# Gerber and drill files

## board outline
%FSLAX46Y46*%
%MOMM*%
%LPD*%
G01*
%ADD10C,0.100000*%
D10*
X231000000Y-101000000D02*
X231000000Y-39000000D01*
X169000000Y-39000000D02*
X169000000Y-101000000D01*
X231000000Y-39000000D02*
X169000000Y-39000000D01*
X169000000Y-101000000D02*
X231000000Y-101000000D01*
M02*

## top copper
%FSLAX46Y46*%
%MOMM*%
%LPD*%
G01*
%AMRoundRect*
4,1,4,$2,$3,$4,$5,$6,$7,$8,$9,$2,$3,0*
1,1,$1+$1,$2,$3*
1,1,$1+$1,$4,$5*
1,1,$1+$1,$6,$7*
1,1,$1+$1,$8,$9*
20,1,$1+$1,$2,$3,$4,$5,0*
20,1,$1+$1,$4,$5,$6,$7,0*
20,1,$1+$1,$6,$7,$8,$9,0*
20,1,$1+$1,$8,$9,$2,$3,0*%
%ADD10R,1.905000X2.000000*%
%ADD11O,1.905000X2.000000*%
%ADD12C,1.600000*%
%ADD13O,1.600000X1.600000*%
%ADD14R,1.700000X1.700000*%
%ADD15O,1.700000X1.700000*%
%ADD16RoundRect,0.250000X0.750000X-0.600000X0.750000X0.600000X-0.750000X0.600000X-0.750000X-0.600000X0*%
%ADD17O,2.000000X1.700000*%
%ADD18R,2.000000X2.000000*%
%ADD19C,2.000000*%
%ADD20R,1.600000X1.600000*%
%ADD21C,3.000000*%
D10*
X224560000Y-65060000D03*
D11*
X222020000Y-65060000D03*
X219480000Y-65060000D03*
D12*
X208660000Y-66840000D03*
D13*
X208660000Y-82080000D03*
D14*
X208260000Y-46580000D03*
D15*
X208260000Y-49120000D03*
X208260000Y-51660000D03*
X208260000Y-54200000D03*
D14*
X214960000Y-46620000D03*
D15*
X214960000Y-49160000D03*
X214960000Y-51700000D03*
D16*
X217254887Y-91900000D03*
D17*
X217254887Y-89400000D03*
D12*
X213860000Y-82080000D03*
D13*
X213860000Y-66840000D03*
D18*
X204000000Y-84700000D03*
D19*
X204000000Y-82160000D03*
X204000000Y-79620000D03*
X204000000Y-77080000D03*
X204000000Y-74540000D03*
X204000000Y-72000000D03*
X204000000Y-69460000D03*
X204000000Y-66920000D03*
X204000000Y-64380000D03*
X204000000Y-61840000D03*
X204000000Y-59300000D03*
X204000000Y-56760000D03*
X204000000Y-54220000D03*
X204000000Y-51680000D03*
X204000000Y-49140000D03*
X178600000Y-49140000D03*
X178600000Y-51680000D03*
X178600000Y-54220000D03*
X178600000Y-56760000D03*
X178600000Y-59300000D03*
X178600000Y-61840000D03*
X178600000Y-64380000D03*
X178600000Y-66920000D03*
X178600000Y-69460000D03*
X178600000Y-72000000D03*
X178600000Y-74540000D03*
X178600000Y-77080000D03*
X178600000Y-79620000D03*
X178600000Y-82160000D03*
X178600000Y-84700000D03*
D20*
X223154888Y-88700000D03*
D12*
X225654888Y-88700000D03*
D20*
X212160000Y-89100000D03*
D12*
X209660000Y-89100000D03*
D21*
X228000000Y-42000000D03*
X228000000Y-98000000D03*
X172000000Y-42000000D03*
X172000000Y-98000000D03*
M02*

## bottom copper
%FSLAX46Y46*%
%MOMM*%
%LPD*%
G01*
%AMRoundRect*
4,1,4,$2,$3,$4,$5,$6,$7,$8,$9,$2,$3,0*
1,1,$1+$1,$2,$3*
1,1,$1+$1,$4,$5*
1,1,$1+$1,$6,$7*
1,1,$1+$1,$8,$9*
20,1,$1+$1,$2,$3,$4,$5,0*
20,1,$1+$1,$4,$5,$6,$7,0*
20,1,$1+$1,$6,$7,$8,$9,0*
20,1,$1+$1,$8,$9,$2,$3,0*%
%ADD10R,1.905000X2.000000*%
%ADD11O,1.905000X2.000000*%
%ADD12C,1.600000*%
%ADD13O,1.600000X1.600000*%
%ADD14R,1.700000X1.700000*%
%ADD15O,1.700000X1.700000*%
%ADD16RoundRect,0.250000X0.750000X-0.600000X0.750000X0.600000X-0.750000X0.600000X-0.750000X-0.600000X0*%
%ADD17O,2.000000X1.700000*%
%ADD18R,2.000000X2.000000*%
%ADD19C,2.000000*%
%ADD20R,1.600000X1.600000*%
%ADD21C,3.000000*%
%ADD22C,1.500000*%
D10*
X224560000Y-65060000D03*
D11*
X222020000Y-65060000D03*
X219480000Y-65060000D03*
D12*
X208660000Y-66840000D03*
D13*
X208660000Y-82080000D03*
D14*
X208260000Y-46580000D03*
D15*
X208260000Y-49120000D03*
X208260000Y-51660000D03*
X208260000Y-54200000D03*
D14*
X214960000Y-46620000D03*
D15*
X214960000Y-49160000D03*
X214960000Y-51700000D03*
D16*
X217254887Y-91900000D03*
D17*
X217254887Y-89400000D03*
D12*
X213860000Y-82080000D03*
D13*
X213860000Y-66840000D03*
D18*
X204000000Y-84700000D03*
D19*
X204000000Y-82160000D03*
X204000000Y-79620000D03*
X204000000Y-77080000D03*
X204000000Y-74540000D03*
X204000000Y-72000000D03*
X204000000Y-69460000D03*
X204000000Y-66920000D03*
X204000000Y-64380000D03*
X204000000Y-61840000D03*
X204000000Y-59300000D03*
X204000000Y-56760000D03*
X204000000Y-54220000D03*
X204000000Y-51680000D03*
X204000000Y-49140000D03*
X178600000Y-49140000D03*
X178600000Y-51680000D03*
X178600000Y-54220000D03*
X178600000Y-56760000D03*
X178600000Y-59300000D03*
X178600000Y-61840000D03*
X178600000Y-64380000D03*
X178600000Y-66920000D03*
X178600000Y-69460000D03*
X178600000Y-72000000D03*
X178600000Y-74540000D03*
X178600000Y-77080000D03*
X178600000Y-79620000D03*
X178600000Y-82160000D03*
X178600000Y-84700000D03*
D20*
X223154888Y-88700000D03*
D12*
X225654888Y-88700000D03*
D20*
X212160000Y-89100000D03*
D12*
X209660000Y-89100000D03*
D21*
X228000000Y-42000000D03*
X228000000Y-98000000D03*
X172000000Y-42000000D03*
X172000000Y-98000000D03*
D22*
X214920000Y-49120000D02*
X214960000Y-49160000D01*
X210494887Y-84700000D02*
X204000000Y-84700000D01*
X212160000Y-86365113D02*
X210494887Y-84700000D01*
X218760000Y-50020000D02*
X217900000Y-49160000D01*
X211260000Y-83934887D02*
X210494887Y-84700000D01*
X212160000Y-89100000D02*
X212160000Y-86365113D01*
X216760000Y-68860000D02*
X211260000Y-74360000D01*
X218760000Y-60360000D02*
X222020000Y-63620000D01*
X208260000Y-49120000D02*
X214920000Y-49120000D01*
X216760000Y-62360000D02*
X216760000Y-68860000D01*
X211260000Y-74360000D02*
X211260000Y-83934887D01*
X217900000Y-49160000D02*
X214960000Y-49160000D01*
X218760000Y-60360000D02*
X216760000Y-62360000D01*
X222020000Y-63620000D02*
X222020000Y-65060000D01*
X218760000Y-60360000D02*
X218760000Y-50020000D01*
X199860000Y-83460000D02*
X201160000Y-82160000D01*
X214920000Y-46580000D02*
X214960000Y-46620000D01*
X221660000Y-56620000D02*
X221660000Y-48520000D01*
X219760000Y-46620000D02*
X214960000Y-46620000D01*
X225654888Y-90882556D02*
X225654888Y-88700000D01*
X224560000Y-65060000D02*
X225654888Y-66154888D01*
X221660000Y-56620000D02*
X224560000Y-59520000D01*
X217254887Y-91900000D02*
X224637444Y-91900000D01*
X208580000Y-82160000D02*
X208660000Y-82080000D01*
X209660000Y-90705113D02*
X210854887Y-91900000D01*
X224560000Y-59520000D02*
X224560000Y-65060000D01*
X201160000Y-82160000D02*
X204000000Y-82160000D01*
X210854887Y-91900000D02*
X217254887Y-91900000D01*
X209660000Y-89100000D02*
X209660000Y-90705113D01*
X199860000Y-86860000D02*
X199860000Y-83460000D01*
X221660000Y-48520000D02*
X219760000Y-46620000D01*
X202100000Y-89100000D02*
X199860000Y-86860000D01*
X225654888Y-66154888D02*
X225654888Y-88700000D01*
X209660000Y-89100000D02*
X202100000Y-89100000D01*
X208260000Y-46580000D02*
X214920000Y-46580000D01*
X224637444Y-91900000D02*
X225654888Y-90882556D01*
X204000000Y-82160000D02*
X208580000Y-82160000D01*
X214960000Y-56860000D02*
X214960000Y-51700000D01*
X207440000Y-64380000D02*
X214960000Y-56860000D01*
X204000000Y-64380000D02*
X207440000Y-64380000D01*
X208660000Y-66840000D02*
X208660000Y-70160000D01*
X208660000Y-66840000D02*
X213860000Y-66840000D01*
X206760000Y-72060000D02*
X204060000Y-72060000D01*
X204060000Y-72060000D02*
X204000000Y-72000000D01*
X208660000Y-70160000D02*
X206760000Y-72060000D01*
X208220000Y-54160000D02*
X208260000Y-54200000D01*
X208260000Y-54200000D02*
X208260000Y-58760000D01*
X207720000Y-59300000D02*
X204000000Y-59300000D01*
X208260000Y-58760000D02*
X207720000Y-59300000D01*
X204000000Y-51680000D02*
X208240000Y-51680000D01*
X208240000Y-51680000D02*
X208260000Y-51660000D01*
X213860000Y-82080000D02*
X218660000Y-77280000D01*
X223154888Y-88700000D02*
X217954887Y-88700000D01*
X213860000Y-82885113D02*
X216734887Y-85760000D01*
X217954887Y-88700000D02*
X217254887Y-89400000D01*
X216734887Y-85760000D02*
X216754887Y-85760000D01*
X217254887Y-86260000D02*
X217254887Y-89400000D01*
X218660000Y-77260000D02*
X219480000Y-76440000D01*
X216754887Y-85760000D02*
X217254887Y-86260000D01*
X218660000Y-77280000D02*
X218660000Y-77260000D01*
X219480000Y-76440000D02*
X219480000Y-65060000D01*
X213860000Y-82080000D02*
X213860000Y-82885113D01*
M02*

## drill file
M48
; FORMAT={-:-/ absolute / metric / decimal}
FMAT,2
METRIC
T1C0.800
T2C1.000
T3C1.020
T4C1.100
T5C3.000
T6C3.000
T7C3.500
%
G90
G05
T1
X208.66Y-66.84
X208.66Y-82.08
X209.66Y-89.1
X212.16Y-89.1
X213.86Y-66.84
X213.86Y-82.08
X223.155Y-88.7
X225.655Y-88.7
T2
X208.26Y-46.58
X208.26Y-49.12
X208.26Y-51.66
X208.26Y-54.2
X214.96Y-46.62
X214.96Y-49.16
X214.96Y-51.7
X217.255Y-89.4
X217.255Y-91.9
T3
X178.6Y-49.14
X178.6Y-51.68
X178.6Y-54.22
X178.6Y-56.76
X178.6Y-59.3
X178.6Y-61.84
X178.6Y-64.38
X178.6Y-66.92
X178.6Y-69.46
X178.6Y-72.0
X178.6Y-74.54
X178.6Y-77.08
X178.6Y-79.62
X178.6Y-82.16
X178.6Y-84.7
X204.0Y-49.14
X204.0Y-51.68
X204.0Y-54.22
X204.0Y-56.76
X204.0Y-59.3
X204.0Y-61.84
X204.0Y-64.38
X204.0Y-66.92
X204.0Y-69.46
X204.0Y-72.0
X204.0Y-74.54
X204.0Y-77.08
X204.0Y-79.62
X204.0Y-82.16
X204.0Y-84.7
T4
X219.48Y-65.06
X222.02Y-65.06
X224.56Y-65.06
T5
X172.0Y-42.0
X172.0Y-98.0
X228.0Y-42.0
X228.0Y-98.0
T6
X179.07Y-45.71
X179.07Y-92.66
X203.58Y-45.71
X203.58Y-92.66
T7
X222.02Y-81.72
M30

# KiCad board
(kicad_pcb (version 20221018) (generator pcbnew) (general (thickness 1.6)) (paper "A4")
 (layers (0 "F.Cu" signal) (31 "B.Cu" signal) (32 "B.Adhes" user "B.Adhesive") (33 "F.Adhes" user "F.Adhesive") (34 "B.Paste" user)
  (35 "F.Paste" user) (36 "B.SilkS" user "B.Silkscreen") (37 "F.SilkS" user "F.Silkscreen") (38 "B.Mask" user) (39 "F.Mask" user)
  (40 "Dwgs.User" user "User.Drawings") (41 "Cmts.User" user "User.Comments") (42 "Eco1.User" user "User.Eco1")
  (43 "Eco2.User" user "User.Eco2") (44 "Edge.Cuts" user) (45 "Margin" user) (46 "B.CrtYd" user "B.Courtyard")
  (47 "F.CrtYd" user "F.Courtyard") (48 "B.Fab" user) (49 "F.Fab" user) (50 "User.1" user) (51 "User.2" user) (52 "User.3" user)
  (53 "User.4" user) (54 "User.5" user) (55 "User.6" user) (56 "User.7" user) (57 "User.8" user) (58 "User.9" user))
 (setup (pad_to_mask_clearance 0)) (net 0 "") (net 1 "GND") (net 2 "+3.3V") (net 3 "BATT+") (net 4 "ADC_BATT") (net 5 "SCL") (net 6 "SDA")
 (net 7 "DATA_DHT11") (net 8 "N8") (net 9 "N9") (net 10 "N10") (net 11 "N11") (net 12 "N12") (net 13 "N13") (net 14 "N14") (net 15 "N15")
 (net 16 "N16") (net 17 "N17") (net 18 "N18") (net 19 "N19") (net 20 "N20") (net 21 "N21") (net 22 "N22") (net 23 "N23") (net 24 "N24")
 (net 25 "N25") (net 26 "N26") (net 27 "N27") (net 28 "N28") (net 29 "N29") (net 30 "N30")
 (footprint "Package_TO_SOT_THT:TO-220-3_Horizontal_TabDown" (layer "F.Cu") (at 224.56 65.06 180)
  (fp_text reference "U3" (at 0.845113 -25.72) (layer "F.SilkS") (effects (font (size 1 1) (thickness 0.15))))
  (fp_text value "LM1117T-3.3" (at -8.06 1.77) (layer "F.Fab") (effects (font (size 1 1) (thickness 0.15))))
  (pad "" np_thru_hole oval (at 2.54 -16.66 180) (size 3.5 3.5) (drill 3.5) (layers "*.Cu" "*.Mask"))
  (pad "1" thru_hole rect (at 0 0 180) (size 1.905 2) (drill 1.1) (layers "*.Cu" "*.Mask") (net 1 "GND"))
  (pad "2" thru_hole oval (at 2.54 0 180) (size 1.905 2) (drill 1.1) (layers "*.Cu" "*.Mask") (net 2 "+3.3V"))
  (pad "3" thru_hole oval (at 5.08 0 180) (size 1.905 2) (drill 1.1) (layers "*.Cu" "*.Mask") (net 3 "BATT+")))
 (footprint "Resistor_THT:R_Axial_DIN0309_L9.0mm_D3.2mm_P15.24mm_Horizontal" (layer "F.Cu") (at 208.66 66.84 -90)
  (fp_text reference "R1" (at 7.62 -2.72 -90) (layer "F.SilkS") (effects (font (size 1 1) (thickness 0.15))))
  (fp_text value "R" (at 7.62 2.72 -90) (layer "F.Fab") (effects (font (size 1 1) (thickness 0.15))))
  (pad "1" thru_hole circle (at 0 0 270) (size 1.6 1.6) (drill 0.8) (layers "*.Cu" "*.Mask") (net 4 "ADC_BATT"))
  (pad "2" thru_hole oval (at 15.24 0 270) (size 1.6 1.6) (drill 0.8) (layers "*.Cu" "*.Mask") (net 1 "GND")))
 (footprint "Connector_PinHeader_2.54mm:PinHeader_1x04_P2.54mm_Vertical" (layer "F.Cu") (at 208.26 46.58)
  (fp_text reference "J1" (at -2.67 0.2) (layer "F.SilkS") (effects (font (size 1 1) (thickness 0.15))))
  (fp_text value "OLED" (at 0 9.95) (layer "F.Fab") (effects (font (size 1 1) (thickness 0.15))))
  (pad "1" thru_hole rect (at 0 0) (size 1.7 1.7) (drill 1) (layers "*.Cu" "*.Mask") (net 1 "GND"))
  (pad "2" thru_hole oval (at 0 2.54) (size 1.7 1.7) (drill 1) (layers "*.Cu" "*.Mask") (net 2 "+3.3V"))
  (pad "3" thru_hole oval (at 0 5.08) (size 1.7 1.7) (drill 1) (layers "*.Cu" "*.Mask") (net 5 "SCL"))
  (pad "4" thru_hole oval (at 0 7.62) (size 1.7 1.7) (drill 1) (layers "*.Cu" "*.Mask") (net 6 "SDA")))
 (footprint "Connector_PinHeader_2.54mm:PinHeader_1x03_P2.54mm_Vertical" (layer "F.Cu") (at 214.96 46.62)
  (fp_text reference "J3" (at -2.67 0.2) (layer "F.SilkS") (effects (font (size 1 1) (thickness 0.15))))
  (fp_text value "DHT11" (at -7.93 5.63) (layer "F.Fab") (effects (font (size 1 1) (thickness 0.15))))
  (pad "1" thru_hole rect (at 0 0) (size 1.7 1.7) (drill 1) (layers "*.Cu" "*.Mask") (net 1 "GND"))
  (pad "2" thru_hole oval (at 0 2.54) (size 1.7 1.7) (drill 1) (layers "*.Cu" "*.Mask") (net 2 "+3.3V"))
  (pad "3" thru_hole oval (at 0 5.08) (size 1.7 1.7) (drill 1) (layers "*.Cu" "*.Mask") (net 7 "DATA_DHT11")))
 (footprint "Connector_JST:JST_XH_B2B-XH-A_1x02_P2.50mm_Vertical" (layer "F.Cu") (at 217.254887 91.9 90)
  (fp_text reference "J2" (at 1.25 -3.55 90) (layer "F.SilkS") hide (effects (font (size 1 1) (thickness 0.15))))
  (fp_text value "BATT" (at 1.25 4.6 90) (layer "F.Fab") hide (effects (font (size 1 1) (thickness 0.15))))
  (pad "1" thru_hole roundrect (at 0 0 90) (size 1.7 2) (drill 1) (layers "*.Cu" "*.Mask") (roundrect_rratio 0.1470588235) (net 1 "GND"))
  (pad "2" thru_hole oval (at 2.5 0 90) (size 1.7 2) (drill 1) (layers "*.Cu" "*.Mask") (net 3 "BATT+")))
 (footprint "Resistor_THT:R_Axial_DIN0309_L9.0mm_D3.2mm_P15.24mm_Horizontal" (layer "F.Cu") (at 213.86 82.08 90)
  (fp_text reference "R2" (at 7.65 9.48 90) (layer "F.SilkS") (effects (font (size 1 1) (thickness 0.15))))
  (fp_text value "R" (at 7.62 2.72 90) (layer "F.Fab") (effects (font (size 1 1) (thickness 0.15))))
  (pad "1" thru_hole circle (at 0 0 90) (size 1.6 1.6) (drill 0.8) (layers "*.Cu" "*.Mask") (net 3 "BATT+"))
  (pad "2" thru_hole oval (at 15.24 0 90) (size 1.6 1.6) (drill 0.8) (layers "*.Cu" "*.Mask") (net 4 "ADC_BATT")))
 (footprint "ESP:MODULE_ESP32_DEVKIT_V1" (layer "F.Cu") (at 191.3 69.185 180)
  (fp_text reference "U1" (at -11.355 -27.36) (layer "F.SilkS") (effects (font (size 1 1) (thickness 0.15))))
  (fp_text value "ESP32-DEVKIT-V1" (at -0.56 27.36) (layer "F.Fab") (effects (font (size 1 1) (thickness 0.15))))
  (pad "" np_thru_hole circle (at -12.28 -23.475 180) (size 3 3) (drill 3) (layers "*.Cu" "*.Mask"))
  (pad "" np_thru_hole circle (at -12.28 23.475 180) (size 3 3) (drill 3) (layers "*.Cu" "*.Mask"))
  (pad "" np_thru_hole circle (at 12.23 -23.475 180) (size 3 3) (drill 3) (layers "*.Cu" "*.Mask"))
  (pad "" np_thru_hole circle (at 12.23 23.475 180) (size 3 3) (drill 3) (layers "*.Cu" "*.Mask"))
  (pad "1" thru_hole rect (at -12.7 -15.515 180) (size 2 2) (drill 1.02) (layers "*.Cu" "*.Mask") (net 2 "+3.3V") (solder_mask_margin 0.102))
  (pad "2" thru_hole circle (at -12.7 -12.975 180) (size 2 2) (drill 1.02) (layers "*.Cu" "*.Mask") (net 1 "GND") (solder_mask_margin 0.102))
  (pad "3" thru_hole circle (at -12.7 -10.435 180) (size 2 2) (drill 1.02) (layers "*.Cu" "*.Mask") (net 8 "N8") (solder_mask_margin 0.102))
  (pad "4" thru_hole circle (at -12.7 -7.895 180) (size 2 2) (drill 1.02) (layers "*.Cu" "*.Mask") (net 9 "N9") (solder_mask_margin 0.102))
  (pad "5" thru_hole circle (at -12.7 -5.355 180) (size 2 2) (drill 1.02) (layers "*.Cu" "*.Mask") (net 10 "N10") (solder_mask_margin 0.102))
  (pad "6" thru_hole circle (at -12.7 -2.815 180) (size 2 2) (drill 1.02) (layers "*.Cu" "*.Mask") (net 4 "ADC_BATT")
   (solder_mask_margin 0.102))
  (pad "7" thru_hole circle (at -12.7 -0.275 180) (size 2 2) (drill 1.02) (layers "*.Cu" "*.Mask") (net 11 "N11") (solder_mask_margin 0.102))
  (pad "8" thru_hole circle (at -12.7 2.265 180) (size 2 2) (drill 1.02) (layers "*.Cu" "*.Mask") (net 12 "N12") (solder_mask_margin 0.102))
  (pad "9" thru_hole circle (at -12.7 4.805 180) (size 2 2) (drill 1.02) (layers "*.Cu" "*.Mask") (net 7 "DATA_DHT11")
   (solder_mask_margin 0.102))
  (pad "10" thru_hole circle (at -12.7 7.345 180) (size 2 2) (drill 1.02) (layers "*.Cu" "*.Mask") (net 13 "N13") (solder_mask_margin 0.102))
  (pad "11" thru_hole circle (at -12.7 9.885 180) (size 2 2) (drill 1.02) (layers "*.Cu" "*.Mask") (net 6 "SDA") (solder_mask_margin 0.102))
  (pad "12" thru_hole circle (at -12.7 12.425 180) (size 2 2) (drill 1.02) (layers "*.Cu" "*.Mask") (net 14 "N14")
   (solder_mask_margin 0.102))
  (pad "13" thru_hole circle (at -12.7 14.965 180) (size 2 2) (drill 1.02) (layers "*.Cu" "*.Mask") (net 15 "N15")
   (solder_mask_margin 0.102))
  (pad "14" thru_hole circle (at -12.7 17.505 180) (size 2 2) (drill 1.02) (layers "*.Cu" "*.Mask") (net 5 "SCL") (solder_mask_margin 0.102))
  (pad "15" thru_hole circle (at -12.7 20.045 180) (size 2 2) (drill 1.02) (layers "*.Cu" "*.Mask") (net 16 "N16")
   (solder_mask_margin 0.102))
  (pad "16" thru_hole circle (at 12.7 20.045 180) (size 2 2) (drill 1.02) (layers "*.Cu" "*.Mask") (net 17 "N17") (solder_mask_margin 0.102))
  (pad "17" thru_hole circle (at 12.7 17.505 180) (size 2 2) (drill 1.02) (layers "*.Cu" "*.Mask") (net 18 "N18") (solder_mask_margin 0.102))
  (pad "18" thru_hole circle (at 12.7 14.965 180) (size 2 2) (drill 1.02) (layers "*.Cu" "*.Mask") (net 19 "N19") (solder_mask_margin 0.102))
  (pad "19" thru_hole circle (at 12.7 12.425 180) (size 2 2) (drill 1.02) (layers "*.Cu" "*.Mask") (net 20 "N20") (solder_mask_margin 0.102))
  (pad "20" thru_hole circle (at 12.7 9.885 180) (size 2 2) (drill 1.02) (layers "*.Cu" "*.Mask") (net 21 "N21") (solder_mask_margin 0.102))
  (pad "21" thru_hole circle (at 12.7 7.345 180) (size 2 2) (drill 1.02) (layers "*.Cu" "*.Mask") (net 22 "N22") (solder_mask_margin 0.102))
  (pad "22" thru_hole circle (at 12.7 4.805 180) (size 2 2) (drill 1.02) (layers "*.Cu" "*.Mask") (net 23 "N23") (solder_mask_margin 0.102))
  (pad "23" thru_hole circle (at 12.7 2.265 180) (size 2 2) (drill 1.02) (layers "*.Cu" "*.Mask") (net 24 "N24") (solder_mask_margin 0.102))
  (pad "24" thru_hole circle (at 12.7 -0.275 180) (size 2 2) (drill 1.02) (layers "*.Cu" "*.Mask") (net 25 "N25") (solder_mask_margin 0.102))
  (pad "25" thru_hole circle (at 12.7 -2.815 180) (size 2 2) (drill 1.02) (layers "*.Cu" "*.Mask") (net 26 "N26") (solder_mask_margin 0.102))
  (pad "26" thru_hole circle (at 12.7 -5.355 180) (size 2 2) (drill 1.02) (layers "*.Cu" "*.Mask") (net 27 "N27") (solder_mask_margin 0.102))
  (pad "27" thru_hole circle (at 12.7 -7.895 180) (size 2 2) (drill 1.02) (layers "*.Cu" "*.Mask") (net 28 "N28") (solder_mask_margin 0.102))
  (pad "28" thru_hole circle (at 12.7 -10.435 180) (size 2 2) (drill 1.02) (layers "*.Cu" "*.Mask") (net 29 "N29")
   (solder_mask_margin 0.102))
  (pad "29" thru_hole circle (at 12.7 -12.975 180) (size 2 2) (drill 1.02) (layers "*.Cu" "*.Mask") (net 1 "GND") (solder_mask_margin 0.102))
  (pad "30" thru_hole circle (at 12.7 -15.515 180) (size 2 2) (drill 1.02) (layers "*.Cu" "*.Mask") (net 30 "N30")
   (solder_mask_margin 0.102))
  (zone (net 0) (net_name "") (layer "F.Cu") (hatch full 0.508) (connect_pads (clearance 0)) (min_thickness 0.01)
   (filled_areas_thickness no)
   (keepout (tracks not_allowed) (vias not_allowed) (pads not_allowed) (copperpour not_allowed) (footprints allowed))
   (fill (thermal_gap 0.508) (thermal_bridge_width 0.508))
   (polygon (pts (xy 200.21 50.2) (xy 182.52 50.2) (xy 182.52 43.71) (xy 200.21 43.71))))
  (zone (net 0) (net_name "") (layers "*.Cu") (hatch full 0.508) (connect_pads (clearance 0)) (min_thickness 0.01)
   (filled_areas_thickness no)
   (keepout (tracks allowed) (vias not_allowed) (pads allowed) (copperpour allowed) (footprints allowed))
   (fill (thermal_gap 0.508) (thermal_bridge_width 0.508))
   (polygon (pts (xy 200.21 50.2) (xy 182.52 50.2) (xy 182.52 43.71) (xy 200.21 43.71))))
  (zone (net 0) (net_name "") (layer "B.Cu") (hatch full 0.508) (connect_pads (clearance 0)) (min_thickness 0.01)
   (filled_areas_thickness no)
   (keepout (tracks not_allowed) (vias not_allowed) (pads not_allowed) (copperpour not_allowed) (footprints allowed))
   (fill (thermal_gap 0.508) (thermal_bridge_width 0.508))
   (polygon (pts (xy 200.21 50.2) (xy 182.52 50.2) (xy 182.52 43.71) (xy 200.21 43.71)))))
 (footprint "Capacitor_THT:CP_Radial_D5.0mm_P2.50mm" (layer "F.Cu") (at 223.154888 88.7)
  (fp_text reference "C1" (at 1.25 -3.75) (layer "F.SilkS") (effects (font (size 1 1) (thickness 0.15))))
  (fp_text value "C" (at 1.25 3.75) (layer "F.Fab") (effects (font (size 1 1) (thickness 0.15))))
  (pad "1" thru_hole rect (at 0 0) (size 1.6 1.6) (drill 0.8) (layers "*.Cu" "*.Mask") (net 3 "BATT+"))
  (pad "2" thru_hole circle (at 2.5 0) (size 1.6 1.6) (drill 0.8) (layers "*.Cu" "*.Mask") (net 1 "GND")))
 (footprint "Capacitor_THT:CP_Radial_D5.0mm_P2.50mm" (layer "F.Cu") (at 212.16 89.1 180)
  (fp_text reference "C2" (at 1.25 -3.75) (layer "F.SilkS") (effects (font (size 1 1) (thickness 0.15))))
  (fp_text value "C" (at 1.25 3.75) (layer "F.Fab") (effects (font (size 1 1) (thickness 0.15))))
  (pad "1" thru_hole rect (at 0 0 180) (size 1.6 1.6) (drill 0.8) (layers "*.Cu" "*.Mask") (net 2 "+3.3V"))
  (pad "2" thru_hole circle (at 2.5 0 180) (size 1.6 1.6) (drill 0.8) (layers "*.Cu" "*.Mask") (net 1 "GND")))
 (gr_line (start 231 101) (end 231 39) (stroke (width 0.1) (type default)) (layer "Edge.Cuts"))
 (gr_line (start 169 39) (end 169 101) (stroke (width 0.1) (type default)) (layer "Edge.Cuts"))
 (gr_line (start 231 39) (end 169 39) (stroke (width 0.1) (type default)) (layer "Edge.Cuts"))
 (gr_line (start 169 101) (end 231 101) (stroke (width 0.1) (type default)) (layer "Edge.Cuts"))
 (via (at 228 42) (size 3) (drill 3) (layers "F.Cu" "B.Cu") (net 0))
 (via (at 228 98) (size 3) (drill 3) (layers "F.Cu" "B.Cu") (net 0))
 (via (at 172 42) (size 3) (drill 3) (layers "F.Cu" "B.Cu") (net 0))
 (via (at 172 98) (size 3) (drill 3) (layers "F.Cu" "B.Cu") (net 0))
 (segment (start 214.92 49.12) (end 214.96 49.16) (width 1.5) (layer "B.Cu") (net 2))
 (segment (start 210.494887 84.7) (end 204 84.7) (width 1.5) (layer "B.Cu") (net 2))
 (segment (start 212.16 86.365113) (end 210.494887 84.7) (width 1.5) (layer "B.Cu") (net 2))
 (segment (start 218.76 50.02) (end 217.9 49.16) (width 1.5) (layer "B.Cu") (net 2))
 (segment (start 211.26 83.934887) (end 210.494887 84.7) (width 1.5) (layer "B.Cu") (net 2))
 (segment (start 212.16 89.1) (end 212.16 86.365113) (width 1.5) (layer "B.Cu") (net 2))
 (segment (start 216.76 68.86) (end 211.26 74.36) (width 1.5) (layer "B.Cu") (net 2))
 (segment (start 218.76 60.36) (end 222.02 63.62) (width 1.5) (layer "B.Cu") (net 2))
 (segment (start 208.26 49.12) (end 214.92 49.12) (width 1.5) (layer "B.Cu") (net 2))
 (segment (start 216.76 62.36) (end 216.76 68.86) (width 1.5) (layer "B.Cu") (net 2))
 (segment (start 211.26 74.36) (end 211.26 83.934887) (width 1.5) (layer "B.Cu") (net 2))
 (segment (start 217.9 49.16) (end 214.96 49.16) (width 1.5) (layer "B.Cu") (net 2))
 (segment (start 218.76 60.36) (end 216.76 62.36) (width 1.5) (layer "B.Cu") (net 2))
 (segment (start 222.02 63.62) (end 222.02 65.06) (width 1.5) (layer "B.Cu") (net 2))
 (segment (start 218.76 60.36) (end 218.76 50.02) (width 1.5) (layer "B.Cu") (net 2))
 (segment (start 199.86 83.46) (end 201.16 82.16) (width 1.5) (layer "B.Cu") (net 1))
 (segment (start 214.92 46.58) (end 214.96 46.62) (width 1.5) (layer "B.Cu") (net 1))
 (segment (start 221.66 56.62) (end 221.66 48.52) (width 1.5) (layer "B.Cu") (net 1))
 (segment (start 219.76 46.62) (end 214.96 46.62) (width 1.5) (layer "B.Cu") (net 1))
 (segment (start 225.654888 90.882556) (end 225.654888 88.7) (width 1.5) (layer "B.Cu") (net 1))
 (segment (start 224.56 65.06) (end 225.654888 66.154888) (width 1.5) (layer "B.Cu") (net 1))
 (segment (start 221.66 56.62) (end 224.56 59.52) (width 1.5) (layer "B.Cu") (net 1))
 (segment (start 217.254887 91.9) (end 224.637444 91.9) (width 1.5) (layer "B.Cu") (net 1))
 (segment (start 208.58 82.16) (end 208.66 82.08) (width 1.5) (layer "B.Cu") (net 1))
 (segment (start 209.66 90.705113) (end 210.854887 91.9) (width 1.5) (layer "B.Cu") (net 1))
 (segment (start 224.56 59.52) (end 224.56 65.06) (width 1.5) (layer "B.Cu") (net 1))
 (segment (start 201.16 82.16) (end 204 82.16) (width 1.5) (layer "B.Cu") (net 1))
 (segment (start 210.854887 91.9) (end 217.254887 91.9) (width 1.5) (layer "B.Cu") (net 1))
 (segment (start 209.66 89.1) (end 209.66 90.705113) (width 1.5) (layer "B.Cu") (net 1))
 (segment (start 199.86 86.86) (end 199.86 83.46) (width 1.5) (layer "B.Cu") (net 1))
 (segment (start 221.66 48.52) (end 219.76 46.62) (width 1.5) (layer "B.Cu") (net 1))
 (segment (start 202.1 89.1) (end 199.86 86.86) (width 1.5) (layer "B.Cu") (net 1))
 (segment (start 225.654888 66.154888) (end 225.654888 88.7) (width 1.5) (layer "B.Cu") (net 1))
 (segment (start 209.66 89.1) (end 202.1 89.1) (width 1.5) (layer "B.Cu") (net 1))
 (segment (start 208.26 46.58) (end 214.92 46.58) (width 1.5) (layer "B.Cu") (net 1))
 (segment (start 224.637444 91.9) (end 225.654888 90.882556) (width 1.5) (layer "B.Cu") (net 1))
 (segment (start 204 82.16) (end 208.58 82.16) (width 1.5) (layer "B.Cu") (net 1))
 (segment (start 214.96 56.86) (end 214.96 51.7) (width 1.5) (layer "B.Cu") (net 7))
 (segment (start 207.44 64.38) (end 214.96 56.86) (width 1.5) (layer "B.Cu") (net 7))
 (segment (start 204 64.38) (end 207.44 64.38) (width 1.5) (layer "B.Cu") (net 7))
 (segment (start 208.66 66.84) (end 208.66 70.16) (width 1.5) (layer "B.Cu") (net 4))
 (segment (start 208.66 66.84) (end 213.86 66.84) (width 1.5) (layer "B.Cu") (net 4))
 (segment (start 206.76 72.06) (end 204.06 72.06) (width 1.5) (layer "B.Cu") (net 4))
 (segment (start 204.06 72.06) (end 204 72) (width 1.5) (layer "B.Cu") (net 4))
 (segment (start 208.66 70.16) (end 206.76 72.06) (width 1.5) (layer "B.Cu") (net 4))
 (segment (start 208.22 54.16) (end 208.26 54.2) (width 1.5) (layer "B.Cu") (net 6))
 (segment (start 208.26 54.2) (end 208.26 58.76) (width 1.5) (layer "B.Cu") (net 6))
 (segment (start 207.72 59.3) (end 204 59.3) (width 1.5) (layer "B.Cu") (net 6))
 (segment (start 208.26 58.76) (end 207.72 59.3) (width 1.5) (layer "B.Cu") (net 6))
 (segment (start 204 51.68) (end 208.24 51.68) (width 1.5) (layer "B.Cu") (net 5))
 (segment (start 208.24 51.68) (end 208.26 51.66) (width 1.5) (layer "B.Cu") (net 5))
 (segment (start 213.86 82.08) (end 218.66 77.28) (width 1.5) (layer "B.Cu") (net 3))
 (segment (start 223.154888 88.7) (end 217.954887 88.7) (width 1.5) (layer "B.Cu") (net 3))
 (segment (start 213.86 82.885113) (end 216.734887 85.76) (width 1.5) (layer "B.Cu") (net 3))
 (segment (start 217.954887 88.7) (end 217.254887 89.4) (width 1.5) (layer "B.Cu") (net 3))
 (segment (start 216.734887 85.76) (end 216.754887 85.76) (width 1.5) (layer "B.Cu") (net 3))
 (segment (start 217.254887 86.26) (end 217.254887 89.4) (width 1.5) (layer "B.Cu") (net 3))
 (segment (start 218.66 77.26) (end 219.48 76.44) (width 1.5) (layer "B.Cu") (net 3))
 (segment (start 216.754887 85.76) (end 217.254887 86.26) (width 1.5) (layer "B.Cu") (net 3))
 (segment (start 218.66 77.28) (end 218.66 77.26) (width 1.5) (layer "B.Cu") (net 3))
 (segment (start 219.48 76.44) (end 219.48 65.06) (width 1.5) (layer "B.Cu") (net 3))
 (segment (start 213.86 82.08) (end 213.86 82.885113) (width 1.5) (layer "B.Cu") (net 3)))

